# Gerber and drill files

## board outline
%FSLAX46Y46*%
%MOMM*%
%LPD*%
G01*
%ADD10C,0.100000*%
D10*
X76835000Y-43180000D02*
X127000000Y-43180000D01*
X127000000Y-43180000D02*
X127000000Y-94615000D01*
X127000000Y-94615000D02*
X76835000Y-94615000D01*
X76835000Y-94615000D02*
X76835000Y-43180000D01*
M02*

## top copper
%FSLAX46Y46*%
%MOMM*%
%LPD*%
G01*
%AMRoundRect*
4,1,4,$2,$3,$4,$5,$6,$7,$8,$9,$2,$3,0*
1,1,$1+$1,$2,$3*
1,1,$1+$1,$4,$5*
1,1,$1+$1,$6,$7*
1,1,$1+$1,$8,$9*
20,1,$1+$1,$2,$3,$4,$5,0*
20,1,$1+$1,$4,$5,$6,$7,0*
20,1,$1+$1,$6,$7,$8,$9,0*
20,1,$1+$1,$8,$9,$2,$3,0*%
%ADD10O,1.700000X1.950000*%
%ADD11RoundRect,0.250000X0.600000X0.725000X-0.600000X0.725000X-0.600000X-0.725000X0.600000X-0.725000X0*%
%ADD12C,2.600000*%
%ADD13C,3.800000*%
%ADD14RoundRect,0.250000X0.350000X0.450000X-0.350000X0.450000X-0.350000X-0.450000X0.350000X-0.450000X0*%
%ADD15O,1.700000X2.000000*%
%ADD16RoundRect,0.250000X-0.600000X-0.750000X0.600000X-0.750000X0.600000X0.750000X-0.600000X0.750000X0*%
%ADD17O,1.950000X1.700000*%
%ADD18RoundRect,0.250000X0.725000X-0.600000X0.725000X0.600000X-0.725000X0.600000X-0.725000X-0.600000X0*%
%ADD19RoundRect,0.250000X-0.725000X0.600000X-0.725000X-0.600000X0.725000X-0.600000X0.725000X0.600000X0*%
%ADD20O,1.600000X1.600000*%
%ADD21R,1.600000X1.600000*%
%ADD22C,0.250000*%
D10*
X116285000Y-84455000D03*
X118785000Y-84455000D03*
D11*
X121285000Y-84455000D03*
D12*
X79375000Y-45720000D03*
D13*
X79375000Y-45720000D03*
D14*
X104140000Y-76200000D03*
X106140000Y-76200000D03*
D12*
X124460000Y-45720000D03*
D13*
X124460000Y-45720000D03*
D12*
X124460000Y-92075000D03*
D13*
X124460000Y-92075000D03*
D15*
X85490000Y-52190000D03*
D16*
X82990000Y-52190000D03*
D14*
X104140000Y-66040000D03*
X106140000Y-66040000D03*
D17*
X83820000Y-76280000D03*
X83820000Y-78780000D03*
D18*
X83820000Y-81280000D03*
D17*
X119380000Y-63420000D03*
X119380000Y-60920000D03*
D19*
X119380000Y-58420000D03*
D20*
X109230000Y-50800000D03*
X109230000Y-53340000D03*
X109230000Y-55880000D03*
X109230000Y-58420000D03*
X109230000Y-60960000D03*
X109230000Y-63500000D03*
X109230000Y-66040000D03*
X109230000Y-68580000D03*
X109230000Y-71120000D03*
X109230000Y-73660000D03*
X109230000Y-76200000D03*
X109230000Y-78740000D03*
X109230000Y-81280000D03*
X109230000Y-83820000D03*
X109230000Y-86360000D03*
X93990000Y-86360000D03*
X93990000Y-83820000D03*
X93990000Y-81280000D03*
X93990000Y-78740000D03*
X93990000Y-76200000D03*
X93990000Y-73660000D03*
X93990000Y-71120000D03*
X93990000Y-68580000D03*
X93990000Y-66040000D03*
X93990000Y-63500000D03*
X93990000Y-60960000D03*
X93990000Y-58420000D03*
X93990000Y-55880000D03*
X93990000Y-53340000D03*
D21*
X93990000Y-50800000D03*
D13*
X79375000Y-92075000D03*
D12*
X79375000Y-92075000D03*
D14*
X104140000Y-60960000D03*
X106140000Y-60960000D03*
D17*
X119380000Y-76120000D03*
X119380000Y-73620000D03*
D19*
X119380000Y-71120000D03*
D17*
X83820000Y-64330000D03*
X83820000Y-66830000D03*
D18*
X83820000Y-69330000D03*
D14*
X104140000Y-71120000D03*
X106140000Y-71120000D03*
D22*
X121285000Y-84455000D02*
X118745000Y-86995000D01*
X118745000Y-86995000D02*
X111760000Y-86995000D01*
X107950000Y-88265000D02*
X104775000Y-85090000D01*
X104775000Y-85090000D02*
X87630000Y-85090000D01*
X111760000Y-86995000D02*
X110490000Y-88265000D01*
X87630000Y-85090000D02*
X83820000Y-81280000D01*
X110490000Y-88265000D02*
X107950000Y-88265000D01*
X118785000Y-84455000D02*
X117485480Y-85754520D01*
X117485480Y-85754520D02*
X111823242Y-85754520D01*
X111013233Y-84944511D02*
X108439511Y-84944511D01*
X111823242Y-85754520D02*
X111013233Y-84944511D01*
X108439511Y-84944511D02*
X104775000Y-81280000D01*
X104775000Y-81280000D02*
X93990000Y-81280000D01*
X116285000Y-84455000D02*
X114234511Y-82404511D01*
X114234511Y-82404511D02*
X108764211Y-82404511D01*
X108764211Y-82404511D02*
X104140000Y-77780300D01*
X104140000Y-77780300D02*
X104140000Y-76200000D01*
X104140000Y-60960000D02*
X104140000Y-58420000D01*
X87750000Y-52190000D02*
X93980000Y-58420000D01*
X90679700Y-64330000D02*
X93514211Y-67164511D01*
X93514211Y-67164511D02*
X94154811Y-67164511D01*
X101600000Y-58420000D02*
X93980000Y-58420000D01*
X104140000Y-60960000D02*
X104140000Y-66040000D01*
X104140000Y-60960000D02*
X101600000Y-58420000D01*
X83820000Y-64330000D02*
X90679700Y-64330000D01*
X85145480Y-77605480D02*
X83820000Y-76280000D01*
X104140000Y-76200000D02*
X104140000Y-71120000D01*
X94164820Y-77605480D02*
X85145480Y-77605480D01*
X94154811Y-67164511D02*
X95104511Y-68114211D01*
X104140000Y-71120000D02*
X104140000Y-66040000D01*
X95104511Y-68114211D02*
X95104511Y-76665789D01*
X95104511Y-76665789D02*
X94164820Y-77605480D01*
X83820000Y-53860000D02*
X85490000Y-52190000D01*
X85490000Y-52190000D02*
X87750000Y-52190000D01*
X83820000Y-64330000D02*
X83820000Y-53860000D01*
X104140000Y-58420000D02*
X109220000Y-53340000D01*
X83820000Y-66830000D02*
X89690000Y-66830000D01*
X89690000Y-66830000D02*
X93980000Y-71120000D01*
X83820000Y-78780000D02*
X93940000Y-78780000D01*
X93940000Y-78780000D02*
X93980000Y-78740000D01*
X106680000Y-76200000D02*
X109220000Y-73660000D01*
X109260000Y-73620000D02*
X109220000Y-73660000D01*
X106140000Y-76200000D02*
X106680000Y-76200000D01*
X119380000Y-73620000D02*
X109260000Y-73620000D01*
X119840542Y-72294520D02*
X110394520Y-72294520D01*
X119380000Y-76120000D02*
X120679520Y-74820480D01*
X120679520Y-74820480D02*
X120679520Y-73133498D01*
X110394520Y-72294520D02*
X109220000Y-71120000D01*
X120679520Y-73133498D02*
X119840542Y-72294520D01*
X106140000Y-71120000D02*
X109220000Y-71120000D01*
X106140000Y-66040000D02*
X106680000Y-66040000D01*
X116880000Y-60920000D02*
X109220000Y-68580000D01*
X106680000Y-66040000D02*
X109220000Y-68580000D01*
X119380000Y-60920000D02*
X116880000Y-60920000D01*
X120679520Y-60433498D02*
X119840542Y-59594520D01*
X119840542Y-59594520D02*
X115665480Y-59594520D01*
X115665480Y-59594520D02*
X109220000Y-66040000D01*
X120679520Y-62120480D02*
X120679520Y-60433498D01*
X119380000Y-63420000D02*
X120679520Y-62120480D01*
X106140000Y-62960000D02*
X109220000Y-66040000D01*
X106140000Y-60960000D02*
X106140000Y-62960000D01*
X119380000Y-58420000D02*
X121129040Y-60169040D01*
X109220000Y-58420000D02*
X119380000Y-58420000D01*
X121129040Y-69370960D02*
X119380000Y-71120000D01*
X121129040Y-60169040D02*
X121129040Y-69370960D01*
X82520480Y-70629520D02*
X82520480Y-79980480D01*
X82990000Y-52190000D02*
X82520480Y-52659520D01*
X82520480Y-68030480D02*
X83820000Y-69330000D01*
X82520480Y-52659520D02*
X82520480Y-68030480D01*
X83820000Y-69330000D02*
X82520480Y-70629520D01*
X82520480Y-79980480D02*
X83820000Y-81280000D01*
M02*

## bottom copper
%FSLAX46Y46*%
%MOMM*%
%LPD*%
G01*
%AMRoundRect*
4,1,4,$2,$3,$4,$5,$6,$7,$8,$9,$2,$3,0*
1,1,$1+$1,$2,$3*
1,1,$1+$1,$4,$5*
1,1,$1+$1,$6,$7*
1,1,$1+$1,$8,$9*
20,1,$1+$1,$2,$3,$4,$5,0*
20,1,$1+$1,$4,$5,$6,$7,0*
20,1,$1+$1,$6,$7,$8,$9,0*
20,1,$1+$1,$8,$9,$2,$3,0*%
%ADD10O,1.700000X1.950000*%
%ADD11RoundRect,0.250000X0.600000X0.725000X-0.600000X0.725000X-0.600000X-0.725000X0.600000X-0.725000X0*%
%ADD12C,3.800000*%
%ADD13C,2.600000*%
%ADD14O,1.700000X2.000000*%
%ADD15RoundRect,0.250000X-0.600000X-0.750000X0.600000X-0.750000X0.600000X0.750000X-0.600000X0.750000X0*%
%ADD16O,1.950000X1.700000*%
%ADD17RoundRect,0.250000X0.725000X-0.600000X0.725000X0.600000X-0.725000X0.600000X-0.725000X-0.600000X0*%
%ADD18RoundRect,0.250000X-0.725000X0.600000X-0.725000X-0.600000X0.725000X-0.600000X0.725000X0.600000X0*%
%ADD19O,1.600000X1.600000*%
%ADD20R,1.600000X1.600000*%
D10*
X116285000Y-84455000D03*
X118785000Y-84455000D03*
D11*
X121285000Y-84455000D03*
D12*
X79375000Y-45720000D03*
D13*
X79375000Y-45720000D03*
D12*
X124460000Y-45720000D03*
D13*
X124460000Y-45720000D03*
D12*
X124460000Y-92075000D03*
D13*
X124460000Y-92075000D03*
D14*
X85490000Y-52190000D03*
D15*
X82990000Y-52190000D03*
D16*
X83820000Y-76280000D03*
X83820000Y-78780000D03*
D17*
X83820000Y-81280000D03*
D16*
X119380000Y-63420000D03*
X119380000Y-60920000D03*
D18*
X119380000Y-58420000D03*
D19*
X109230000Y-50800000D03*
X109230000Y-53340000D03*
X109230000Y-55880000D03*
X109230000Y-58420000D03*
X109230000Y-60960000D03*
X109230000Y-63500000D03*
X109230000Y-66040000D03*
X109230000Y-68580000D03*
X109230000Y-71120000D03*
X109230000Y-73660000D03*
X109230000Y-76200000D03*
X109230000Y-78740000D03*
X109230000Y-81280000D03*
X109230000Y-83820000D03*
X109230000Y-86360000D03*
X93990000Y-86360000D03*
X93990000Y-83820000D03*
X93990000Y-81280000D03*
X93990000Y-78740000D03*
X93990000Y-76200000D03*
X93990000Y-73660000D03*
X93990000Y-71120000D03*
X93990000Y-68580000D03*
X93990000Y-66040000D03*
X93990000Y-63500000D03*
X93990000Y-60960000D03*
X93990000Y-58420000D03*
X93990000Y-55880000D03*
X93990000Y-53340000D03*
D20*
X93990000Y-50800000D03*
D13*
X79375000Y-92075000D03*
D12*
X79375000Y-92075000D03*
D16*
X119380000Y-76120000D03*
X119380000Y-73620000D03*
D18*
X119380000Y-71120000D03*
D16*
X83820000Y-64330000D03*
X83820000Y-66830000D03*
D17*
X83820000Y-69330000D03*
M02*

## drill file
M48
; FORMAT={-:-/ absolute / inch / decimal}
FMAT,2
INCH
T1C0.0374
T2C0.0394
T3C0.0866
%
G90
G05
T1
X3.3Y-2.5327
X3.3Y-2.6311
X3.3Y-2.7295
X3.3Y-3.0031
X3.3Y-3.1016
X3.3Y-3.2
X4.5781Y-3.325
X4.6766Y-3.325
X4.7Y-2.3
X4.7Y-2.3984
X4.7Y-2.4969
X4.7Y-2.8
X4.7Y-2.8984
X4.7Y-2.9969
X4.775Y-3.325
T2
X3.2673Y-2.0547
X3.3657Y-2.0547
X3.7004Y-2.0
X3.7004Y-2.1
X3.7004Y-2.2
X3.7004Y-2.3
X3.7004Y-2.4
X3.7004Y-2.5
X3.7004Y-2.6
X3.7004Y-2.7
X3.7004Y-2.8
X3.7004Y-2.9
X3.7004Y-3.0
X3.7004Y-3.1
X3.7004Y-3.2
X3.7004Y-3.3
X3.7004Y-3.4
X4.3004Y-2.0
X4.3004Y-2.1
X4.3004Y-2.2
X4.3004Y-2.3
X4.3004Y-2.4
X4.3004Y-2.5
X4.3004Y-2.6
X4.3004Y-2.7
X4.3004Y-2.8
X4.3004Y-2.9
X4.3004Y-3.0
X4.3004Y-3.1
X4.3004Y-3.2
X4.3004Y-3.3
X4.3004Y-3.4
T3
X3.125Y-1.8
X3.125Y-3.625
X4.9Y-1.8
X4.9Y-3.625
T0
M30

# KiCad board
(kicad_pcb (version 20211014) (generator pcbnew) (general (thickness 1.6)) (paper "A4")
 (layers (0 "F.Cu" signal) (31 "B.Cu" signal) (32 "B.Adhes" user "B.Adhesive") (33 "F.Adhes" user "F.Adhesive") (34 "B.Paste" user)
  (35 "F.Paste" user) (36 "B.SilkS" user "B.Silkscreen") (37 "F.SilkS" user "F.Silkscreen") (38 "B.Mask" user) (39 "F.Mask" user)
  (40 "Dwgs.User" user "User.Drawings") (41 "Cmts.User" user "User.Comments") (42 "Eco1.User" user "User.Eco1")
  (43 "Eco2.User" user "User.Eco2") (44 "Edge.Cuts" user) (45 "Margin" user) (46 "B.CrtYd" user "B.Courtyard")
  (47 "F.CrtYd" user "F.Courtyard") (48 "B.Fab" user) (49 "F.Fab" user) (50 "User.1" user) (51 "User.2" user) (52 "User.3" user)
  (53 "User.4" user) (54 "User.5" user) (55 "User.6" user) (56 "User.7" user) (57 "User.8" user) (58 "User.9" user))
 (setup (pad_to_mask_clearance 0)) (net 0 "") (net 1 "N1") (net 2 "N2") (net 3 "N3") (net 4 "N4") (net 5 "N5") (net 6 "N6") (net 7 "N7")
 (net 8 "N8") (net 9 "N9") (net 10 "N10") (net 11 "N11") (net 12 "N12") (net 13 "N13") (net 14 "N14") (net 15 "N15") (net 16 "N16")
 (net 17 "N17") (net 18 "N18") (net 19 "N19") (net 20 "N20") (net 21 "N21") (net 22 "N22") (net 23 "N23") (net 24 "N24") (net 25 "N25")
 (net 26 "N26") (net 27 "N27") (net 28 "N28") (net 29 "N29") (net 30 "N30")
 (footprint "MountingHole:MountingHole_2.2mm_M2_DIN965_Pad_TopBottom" (layer "F.Cu") (at 79.375 45.72)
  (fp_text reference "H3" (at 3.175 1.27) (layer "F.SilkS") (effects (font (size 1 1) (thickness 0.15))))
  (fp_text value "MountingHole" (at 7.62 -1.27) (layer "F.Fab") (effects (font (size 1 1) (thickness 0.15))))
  (pad "1" connect circle (at 0 0) (size 3.8 3.8) (layers "F.Cu" "F.Mask"))
  (pad "1" thru_hole circle (at 0 0) (size 2.6 2.6) (drill 2.2) (layers *.Cu *.Mask))
  (pad "1" connect circle (at 0 0) (size 3.8 3.8) (layers "B.Cu" "B.Mask")))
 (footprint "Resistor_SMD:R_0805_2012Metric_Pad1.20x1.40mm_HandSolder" (layer "F.Cu") (at 105.14 76.2 180)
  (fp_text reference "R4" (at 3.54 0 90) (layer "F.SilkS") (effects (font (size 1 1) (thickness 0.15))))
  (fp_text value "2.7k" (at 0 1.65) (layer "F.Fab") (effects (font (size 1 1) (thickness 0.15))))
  (pad "1" smd roundrect (at -1 0 180) (size 1.2 1.4) (layers "F.Cu" "F.Paste" "F.Mask") (roundrect_rratio 0.2083333333) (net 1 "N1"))
  (pad "2" smd roundrect (at 1 0 180) (size 1.2 1.4) (layers "F.Cu" "F.Paste" "F.Mask") (roundrect_rratio 0.2083333333) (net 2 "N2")))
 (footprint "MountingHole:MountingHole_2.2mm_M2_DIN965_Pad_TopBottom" (layer "F.Cu") (at 124.46 45.72)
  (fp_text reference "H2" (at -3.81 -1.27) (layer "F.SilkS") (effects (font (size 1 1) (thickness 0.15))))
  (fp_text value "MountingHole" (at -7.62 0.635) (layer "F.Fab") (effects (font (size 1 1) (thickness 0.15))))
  (pad "1" connect circle (at 0 0) (size 3.8 3.8) (layers "F.Cu" "F.Mask"))
  (pad "1" thru_hole circle (at 0 0) (size 2.6 2.6) (drill 2.2) (layers *.Cu *.Mask))
  (pad "1" connect circle (at 0 0) (size 3.8 3.8) (layers "B.Cu" "B.Mask")))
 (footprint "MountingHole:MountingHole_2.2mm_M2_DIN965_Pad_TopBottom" (layer "F.Cu") (at 124.46 92.075)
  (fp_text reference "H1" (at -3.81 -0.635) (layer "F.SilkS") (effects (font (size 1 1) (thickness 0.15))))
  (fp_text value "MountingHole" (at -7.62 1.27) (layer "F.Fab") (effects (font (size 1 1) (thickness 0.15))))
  (pad "1" connect circle (at 0 0) (size 3.8 3.8) (layers "F.Cu" "F.Mask"))
  (pad "1" thru_hole circle (at 0 0) (size 2.6 2.6) (drill 2.2) (layers *.Cu *.Mask))
  (pad "1" connect circle (at 0 0) (size 3.8 3.8) (layers "B.Cu" "B.Mask")))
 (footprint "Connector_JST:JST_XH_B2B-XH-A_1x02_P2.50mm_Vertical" (layer "F.Cu") (at 82.99 52.19)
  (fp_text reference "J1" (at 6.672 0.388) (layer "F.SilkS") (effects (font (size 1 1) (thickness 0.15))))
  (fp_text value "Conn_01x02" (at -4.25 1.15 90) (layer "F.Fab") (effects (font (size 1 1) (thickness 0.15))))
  (pad "1" thru_hole roundrect (at 0 0) (size 1.7 2) (drill 1) (layers *.Cu *.Mask) (roundrect_rratio 0.1470588235) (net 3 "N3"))
  (pad "2" thru_hole oval (at 2.5 0) (size 1.7 2) (drill 1) (layers *.Cu *.Mask) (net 2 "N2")))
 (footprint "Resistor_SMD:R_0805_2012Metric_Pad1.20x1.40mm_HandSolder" (layer "F.Cu") (at 105.14 66.04 180)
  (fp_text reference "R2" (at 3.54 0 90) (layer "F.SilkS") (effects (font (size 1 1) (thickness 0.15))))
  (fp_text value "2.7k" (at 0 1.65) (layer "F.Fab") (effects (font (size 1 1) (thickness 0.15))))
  (pad "1" smd roundrect (at -1 0 180) (size 1.2 1.4) (layers "F.Cu" "F.Paste" "F.Mask") (roundrect_rratio 0.2083333333) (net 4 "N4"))
  (pad "2" smd roundrect (at 1 0 180) (size 1.2 1.4) (layers "F.Cu" "F.Paste" "F.Mask") (roundrect_rratio 0.2083333333) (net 2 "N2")))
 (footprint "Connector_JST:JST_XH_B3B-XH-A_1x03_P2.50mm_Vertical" (layer "F.Cu") (at 83.82 81.28 90)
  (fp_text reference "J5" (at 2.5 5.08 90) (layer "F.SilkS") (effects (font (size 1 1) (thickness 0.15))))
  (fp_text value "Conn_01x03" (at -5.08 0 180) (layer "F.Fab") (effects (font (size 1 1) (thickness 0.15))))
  (pad "1" thru_hole roundrect (at 0 0 90) (size 1.7 1.95) (drill 0.95) (layers *.Cu *.Mask) (roundrect_rratio 0.1470588235) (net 3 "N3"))
  (pad "2" thru_hole oval (at 2.5 0 90) (size 1.7 1.95) (drill 0.95) (layers *.Cu *.Mask) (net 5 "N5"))
  (pad "3" thru_hole oval (at 5 0 90) (size 1.7 1.95) (drill 0.95) (layers *.Cu *.Mask) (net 2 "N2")))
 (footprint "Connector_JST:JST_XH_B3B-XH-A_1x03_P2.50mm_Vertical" (layer "F.Cu") (at 119.38 58.42 -90)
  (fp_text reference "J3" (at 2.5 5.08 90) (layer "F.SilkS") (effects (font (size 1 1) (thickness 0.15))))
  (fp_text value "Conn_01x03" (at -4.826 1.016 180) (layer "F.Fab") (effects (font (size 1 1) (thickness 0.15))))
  (pad "1" thru_hole roundrect (at 0 0 270) (size 1.7 1.95) (drill 0.95) (layers *.Cu *.Mask) (roundrect_rratio 0.1470588235) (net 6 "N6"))
  (pad "2" thru_hole oval (at 2.5 0 270) (size 1.7 1.95) (drill 0.95) (layers *.Cu *.Mask) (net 4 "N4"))
  (pad "3" thru_hole oval (at 5 0 270) (size 1.7 1.95) (drill 0.95) (layers *.Cu *.Mask) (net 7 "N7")))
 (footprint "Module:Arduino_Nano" (layer "F.Cu") (at 93.99 50.8)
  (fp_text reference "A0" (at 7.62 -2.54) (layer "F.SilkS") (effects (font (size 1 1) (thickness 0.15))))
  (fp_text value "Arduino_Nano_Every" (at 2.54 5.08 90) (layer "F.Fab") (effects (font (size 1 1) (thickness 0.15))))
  (pad "1" thru_hole rect (at 0 0) (size 1.6 1.6) (drill 1) (layers *.Cu *.Mask) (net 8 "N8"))
  (pad "2" thru_hole oval (at 0 2.54) (size 1.6 1.6) (drill 1) (layers *.Cu *.Mask) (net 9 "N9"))
  (pad "3" thru_hole oval (at 0 5.08) (size 1.6 1.6) (drill 1) (layers *.Cu *.Mask) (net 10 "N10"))
  (pad "4" thru_hole oval (at 0 7.62) (size 1.6 1.6) (drill 1) (layers *.Cu *.Mask) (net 2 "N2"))
  (pad "5" thru_hole oval (at 0 10.16) (size 1.6 1.6) (drill 1) (layers *.Cu *.Mask) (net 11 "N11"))
  (pad "6" thru_hole oval (at 0 12.7) (size 1.6 1.6) (drill 1) (layers *.Cu *.Mask) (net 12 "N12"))
  (pad "7" thru_hole oval (at 0 15.24) (size 1.6 1.6) (drill 1) (layers *.Cu *.Mask) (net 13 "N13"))
  (pad "8" thru_hole oval (at 0 17.78) (size 1.6 1.6) (drill 1) (layers *.Cu *.Mask) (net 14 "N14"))
  (pad "9" thru_hole oval (at 0 20.32) (size 1.6 1.6) (drill 1) (layers *.Cu *.Mask) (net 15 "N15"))
  (pad "10" thru_hole oval (at 0 22.86) (size 1.6 1.6) (drill 1) (layers *.Cu *.Mask) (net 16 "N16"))
  (pad "11" thru_hole oval (at 0 25.4) (size 1.6 1.6) (drill 1) (layers *.Cu *.Mask) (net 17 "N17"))
  (pad "12" thru_hole oval (at 0 27.94) (size 1.6 1.6) (drill 1) (layers *.Cu *.Mask) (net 5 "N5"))
  (pad "13" thru_hole oval (at 0 30.48) (size 1.6 1.6) (drill 1) (layers *.Cu *.Mask) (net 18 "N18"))
  (pad "14" thru_hole oval (at 0 33.02) (size 1.6 1.6) (drill 1) (layers *.Cu *.Mask) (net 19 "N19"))
  (pad "15" thru_hole oval (at 0 35.56) (size 1.6 1.6) (drill 1) (layers *.Cu *.Mask) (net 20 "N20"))
  (pad "16" thru_hole oval (at 15.24 35.56) (size 1.6 1.6) (drill 1) (layers *.Cu *.Mask) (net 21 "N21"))
  (pad "17" thru_hole oval (at 15.24 33.02) (size 1.6 1.6) (drill 1) (layers *.Cu *.Mask) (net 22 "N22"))
  (pad "18" thru_hole oval (at 15.24 30.48) (size 1.6 1.6) (drill 1) (layers *.Cu *.Mask) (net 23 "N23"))
  (pad "19" thru_hole oval (at 15.24 27.94) (size 1.6 1.6) (drill 1) (layers *.Cu *.Mask) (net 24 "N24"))
  (pad "20" thru_hole oval (at 15.24 25.4) (size 1.6 1.6) (drill 1) (layers *.Cu *.Mask) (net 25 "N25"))
  (pad "21" thru_hole oval (at 15.24 22.86) (size 1.6 1.6) (drill 1) (layers *.Cu *.Mask) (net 1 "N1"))
  (pad "22" thru_hole oval (at 15.24 20.32) (size 1.6 1.6) (drill 1) (layers *.Cu *.Mask) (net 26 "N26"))
  (pad "23" thru_hole oval (at 15.24 17.78) (size 1.6 1.6) (drill 1) (layers *.Cu *.Mask) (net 4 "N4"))
  (pad "24" thru_hole oval (at 15.24 15.24) (size 1.6 1.6) (drill 1) (layers *.Cu *.Mask) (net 7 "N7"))
  (pad "25" thru_hole oval (at 15.24 12.7) (size 1.6 1.6) (drill 1) (layers *.Cu *.Mask) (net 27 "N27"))
  (pad "26" thru_hole oval (at 15.24 10.16) (size 1.6 1.6) (drill 1) (layers *.Cu *.Mask) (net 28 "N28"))
  (pad "27" thru_hole oval (at 15.24 7.62) (size 1.6 1.6) (drill 1) (layers *.Cu *.Mask) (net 6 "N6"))
  (pad "28" thru_hole oval (at 15.24 5.08) (size 1.6 1.6) (drill 1) (layers *.Cu *.Mask) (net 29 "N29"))
  (pad "29" thru_hole oval (at 15.24 2.54) (size 1.6 1.6) (drill 1) (layers *.Cu *.Mask) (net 2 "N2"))
  (pad "30" thru_hole oval (at 15.24 0) (size 1.6 1.6) (drill 1) (layers *.Cu *.Mask) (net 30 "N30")))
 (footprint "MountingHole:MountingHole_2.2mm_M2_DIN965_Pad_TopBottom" (layer "F.Cu") (at 79.375 92.075)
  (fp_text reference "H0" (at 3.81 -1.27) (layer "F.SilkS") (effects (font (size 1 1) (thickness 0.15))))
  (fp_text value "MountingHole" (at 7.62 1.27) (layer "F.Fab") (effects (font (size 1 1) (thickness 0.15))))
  (pad "1" connect circle (at 0 0) (size 3.8 3.8) (layers "B.Cu" "B.Mask"))
  (pad "1" thru_hole circle (at 0 0) (size 2.6 2.6) (drill 2.2) (layers *.Cu *.Mask))
  (pad "1" connect circle (at 0 0) (size 3.8 3.8) (layers "F.Cu" "F.Mask")))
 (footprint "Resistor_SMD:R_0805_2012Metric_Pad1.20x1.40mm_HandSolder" (layer "F.Cu") (at 105.14 60.96 180)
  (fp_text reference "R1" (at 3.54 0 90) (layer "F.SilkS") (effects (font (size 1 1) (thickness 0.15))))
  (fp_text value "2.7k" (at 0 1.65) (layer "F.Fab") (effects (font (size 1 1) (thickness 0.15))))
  (pad "1" smd roundrect (at -1 0 180) (size 1.2 1.4) (layers "F.Cu" "F.Paste" "F.Mask") (roundrect_rratio 0.2083333333) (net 7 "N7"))
  (pad "2" smd roundrect (at 1 0 180) (size 1.2 1.4) (layers "F.Cu" "F.Paste" "F.Mask") (roundrect_rratio 0.2083333333) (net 2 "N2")))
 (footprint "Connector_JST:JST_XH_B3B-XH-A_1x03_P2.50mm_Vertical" (layer "F.Cu") (at 119.38 71.12 -90)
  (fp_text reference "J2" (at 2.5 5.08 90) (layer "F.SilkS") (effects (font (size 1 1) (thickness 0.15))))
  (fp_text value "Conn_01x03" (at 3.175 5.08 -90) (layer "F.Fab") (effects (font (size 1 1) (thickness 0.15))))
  (pad "1" thru_hole roundrect (at 0 0 270) (size 1.7 1.95) (drill 0.95) (layers *.Cu *.Mask) (roundrect_rratio 0.1470588235) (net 6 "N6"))
  (pad "2" thru_hole oval (at 2.5 0 270) (size 1.7 1.95) (drill 0.95) (layers *.Cu *.Mask) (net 1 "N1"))
  (pad "3" thru_hole oval (at 5 0 270) (size 1.7 1.95) (drill 0.95) (layers *.Cu *.Mask) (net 26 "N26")))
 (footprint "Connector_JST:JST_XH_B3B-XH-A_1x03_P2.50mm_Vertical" (layer "F.Cu") (at 83.82 69.33 90)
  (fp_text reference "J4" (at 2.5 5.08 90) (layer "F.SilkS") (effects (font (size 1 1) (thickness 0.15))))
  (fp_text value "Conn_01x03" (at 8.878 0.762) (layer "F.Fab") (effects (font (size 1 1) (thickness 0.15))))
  (pad "1" thru_hole roundrect (at 0 0 90) (size 1.7 1.95) (drill 0.95) (layers *.Cu *.Mask) (roundrect_rratio 0.1470588235) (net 3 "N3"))
  (pad "2" thru_hole oval (at 2.5 0 90) (size 1.7 1.95) (drill 0.95) (layers *.Cu *.Mask) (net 15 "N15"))
  (pad "3" thru_hole oval (at 5 0 90) (size 1.7 1.95) (drill 0.95) (layers *.Cu *.Mask) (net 2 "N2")))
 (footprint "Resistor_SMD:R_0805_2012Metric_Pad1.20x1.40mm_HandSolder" (layer "F.Cu") (at 105.14 71.12 180)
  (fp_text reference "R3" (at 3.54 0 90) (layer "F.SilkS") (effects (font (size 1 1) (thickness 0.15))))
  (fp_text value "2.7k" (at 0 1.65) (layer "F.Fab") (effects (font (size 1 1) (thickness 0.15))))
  (pad "1" smd roundrect (at -1 0 180) (size 1.2 1.4) (layers "F.Cu" "F.Paste" "F.Mask") (roundrect_rratio 0.2083333333) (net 26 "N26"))
  (pad "2" smd roundrect (at 1 0 180) (size 1.2 1.4) (layers "F.Cu" "F.Paste" "F.Mask") (roundrect_rratio 0.2083333333) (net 2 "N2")))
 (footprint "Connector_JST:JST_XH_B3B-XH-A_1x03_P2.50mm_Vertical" (layer "F.Cu") (at 121.285 84.455 180)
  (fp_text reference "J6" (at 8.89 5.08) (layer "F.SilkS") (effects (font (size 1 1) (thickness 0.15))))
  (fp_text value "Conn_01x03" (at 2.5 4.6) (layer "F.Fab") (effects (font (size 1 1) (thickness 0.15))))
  (pad "1" thru_hole roundrect (at 0 0 180) (size 1.7 1.95) (drill 0.95) (layers *.Cu *.Mask) (roundrect_rratio 0.1470588235) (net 3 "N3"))
  (pad "2" thru_hole oval (at 2.5 0 180) (size 1.7 1.95) (drill 0.95) (layers *.Cu *.Mask) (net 18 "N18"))
  (pad "3" thru_hole oval (at 5 0 180) (size 1.7 1.95) (drill 0.95) (layers *.Cu *.Mask) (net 2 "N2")))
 (gr_rect (start 76.835 43.18) (end 127 94.615) (layer "Edge.Cuts") (width 0.1) (fill none))
 (segment (start 108.764211 82.404511) (end 104.14 77.7803) (width 0.25) (layer "F.Cu") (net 2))
 (segment (start 114.234511 82.404511) (end 108.764211 82.404511) (width 0.25) (layer "F.Cu") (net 2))
 (segment (start 104.14 60.96) (end 104.14 58.42) (width 0.25) (layer "F.Cu") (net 2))
 (segment (start 87.75 52.19) (end 93.98 58.42) (width 0.25) (layer "F.Cu") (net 2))
 (segment (start 90.6797 64.33) (end 93.514211 67.164511) (width 0.25) (layer "F.Cu") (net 2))
 (segment (start 93.514211 67.164511) (end 94.154811 67.164511) (width 0.25) (layer "F.Cu") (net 2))
 (segment (start 101.6 58.42) (end 93.98 58.42) (width 0.25) (layer "F.Cu") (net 2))
 (segment (start 104.14 60.96) (end 104.14 66.04) (width 0.25) (layer "F.Cu") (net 2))
 (segment (start 104.14 60.96) (end 101.6 58.42) (width 0.25) (layer "F.Cu") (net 2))
 (segment (start 83.82 64.33) (end 90.6797 64.33) (width 0.25) (layer "F.Cu") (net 2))
 (segment (start 85.14548 77.60548) (end 83.82 76.28) (width 0.25) (layer "F.Cu") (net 2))
 (segment (start 104.14 76.2) (end 104.14 71.12) (width 0.25) (layer "F.Cu") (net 2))
 (segment (start 94.16482 77.60548) (end 85.14548 77.60548) (width 0.25) (layer "F.Cu") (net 2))
 (segment (start 94.154811 67.164511) (end 95.104511 68.114211) (width 0.25) (layer "F.Cu") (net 2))
 (segment (start 116.285 84.455) (end 114.234511 82.404511) (width 0.25) (layer "F.Cu") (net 2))
 (segment (start 104.14 71.12) (end 104.14 66.04) (width 0.25) (layer "F.Cu") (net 2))
 (segment (start 95.104511 68.114211) (end 95.104511 76.665789) (width 0.25) (layer "F.Cu") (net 2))
 (segment (start 95.104511 76.665789) (end 94.16482 77.60548) (width 0.25) (layer "F.Cu") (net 2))
 (segment (start 83.82 53.86) (end 85.49 52.19) (width 0.25) (layer "F.Cu") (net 2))
 (segment (start 85.49 52.19) (end 87.75 52.19) (width 0.25) (layer "F.Cu") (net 2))
 (segment (start 104.14 77.7803) (end 104.14 76.2) (width 0.25) (layer "F.Cu") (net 2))
 (segment (start 83.82 64.33) (end 83.82 53.86) (width 0.25) (layer "F.Cu") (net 2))
 (segment (start 104.14 58.42) (end 109.22 53.34) (width 0.25) (layer "F.Cu") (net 2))
 (segment (start 83.82 66.83) (end 89.69 66.83) (width 0.25) (layer "F.Cu") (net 15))
 (segment (start 89.69 66.83) (end 93.98 71.12) (width 0.25) (layer "F.Cu") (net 15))
 (segment (start 83.82 78.78) (end 93.94 78.78) (width 0.25) (layer "F.Cu") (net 5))
 (segment (start 93.94 78.78) (end 93.98 78.74) (width 0.25) (layer "F.Cu") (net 5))
 (segment (start 108.439511 84.944511) (end 104.775 81.28) (width 0.25) (layer "F.Cu") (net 18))
 (segment (start 104.775 81.28) (end 93.99 81.28) (width 0.25) (layer "F.Cu") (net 18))
 (segment (start 118.785 84.455) (end 117.48548 85.75452) (width 0.25) (layer "F.Cu") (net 18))
 (segment (start 111.823242 85.75452) (end 111.013233 84.944511) (width 0.25) (layer "F.Cu") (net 18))
 (segment (start 117.48548 85.75452) (end 111.823242 85.75452) (width 0.25) (layer "F.Cu") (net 18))
 (segment (start 111.013233 84.944511) (end 108.439511 84.944511) (width 0.25) (layer "F.Cu") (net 18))
 (segment (start 106.68 76.2) (end 109.22 73.66) (width 0.25) (layer "F.Cu") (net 1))
 (segment (start 109.26 73.62) (end 109.22 73.66) (width 0.25) (layer "F.Cu") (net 1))
 (segment (start 106.14 76.2) (end 106.68 76.2) (width 0.25) (layer "F.Cu") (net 1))
 (segment (start 119.38 73.62) (end 109.26 73.62) (width 0.25) (layer "F.Cu") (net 1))
 (segment (start 119.840542 72.29452) (end 110.39452 72.29452) (width 0.25) (layer "F.Cu") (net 26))
 (segment (start 119.38 76.12) (end 120.67952 74.82048) (width 0.25) (layer "F.Cu") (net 26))
 (segment (start 120.67952 74.82048) (end 120.67952 73.133498) (width 0.25) (layer "F.Cu") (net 26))
 (segment (start 110.39452 72.29452) (end 109.22 71.12) (width 0.25) (layer "F.Cu") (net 26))
 (segment (start 120.67952 73.133498) (end 119.840542 72.29452) (width 0.25) (layer "F.Cu") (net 26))
 (segment (start 106.14 71.12) (end 109.22 71.12) (width 0.25) (layer "F.Cu") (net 26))
 (segment (start 106.14 66.04) (end 106.68 66.04) (width 0.25) (layer "F.Cu") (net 4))
 (segment (start 116.88 60.92) (end 109.22 68.58) (width 0.25) (layer "F.Cu") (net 4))
 (segment (start 106.68 66.04) (end 109.22 68.58) (width 0.25) (layer "F.Cu") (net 4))
 (segment (start 119.38 60.92) (end 116.88 60.92) (width 0.25) (layer "F.Cu") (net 4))
 (segment (start 120.67952 60.433498) (end 119.840542 59.59452) (width 0.25) (layer "F.Cu") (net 7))
 (segment (start 119.840542 59.59452) (end 115.66548 59.59452) (width 0.25) (layer "F.Cu") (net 7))
 (segment (start 115.66548 59.59452) (end 109.22 66.04) (width 0.25) (layer "F.Cu") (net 7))
 (segment (start 120.67952 62.12048) (end 120.67952 60.433498) (width 0.25) (layer "F.Cu") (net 7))
 (segment (start 119.38 63.42) (end 120.67952 62.12048) (width 0.25) (layer "F.Cu") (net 7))
 (segment (start 106.14 62.96) (end 109.22 66.04) (width 0.25) (layer "F.Cu") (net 7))
 (segment (start 106.14 60.96) (end 106.14 62.96) (width 0.25) (layer "F.Cu") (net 7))
 (segment (start 119.38 58.42) (end 121.12904 60.16904) (width 0.25) (layer "F.Cu") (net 6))
 (segment (start 109.22 58.42) (end 119.38 58.42) (width 0.25) (layer "F.Cu") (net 6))
 (segment (start 121.12904 69.37096) (end 119.38 71.12) (width 0.25) (layer "F.Cu") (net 6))
 (segment (start 121.12904 60.16904) (end 121.12904 69.37096) (width 0.25) (layer "F.Cu") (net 6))
 (segment (start 82.52048 70.62952) (end 82.52048 79.98048) (width 0.25) (layer "F.Cu") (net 3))
 (segment (start 87.63 85.09) (end 83.82 81.28) (width 0.25) (layer "F.Cu") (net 3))
 (segment (start 82.99 52.19) (end 82.52048 52.65952) (width 0.25) (layer "F.Cu") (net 3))
 (segment (start 121.285 84.455) (end 118.745 86.995) (width 0.25) (layer "F.Cu") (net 3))
 (segment (start 82.52048 68.03048) (end 83.82 69.33) (width 0.25) (layer "F.Cu") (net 3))
 (segment (start 82.52048 52.65952) (end 82.52048 68.03048) (width 0.25) (layer "F.Cu") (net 3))
 (segment (start 83.82 69.33) (end 82.52048 70.62952) (width 0.25) (layer "F.Cu") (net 3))
 (segment (start 110.49 88.265) (end 107.95 88.265) (width 0.25) (layer "F.Cu") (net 3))
 (segment (start 111.76 86.995) (end 110.49 88.265) (width 0.25) (layer "F.Cu") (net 3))
 (segment (start 82.52048 79.98048) (end 83.82 81.28) (width 0.25) (layer "F.Cu") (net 3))
 (segment (start 104.775 85.09) (end 87.63 85.09) (width 0.25) (layer "F.Cu") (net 3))
 (segment (start 118.745 86.995) (end 111.76 86.995) (width 0.25) (layer "F.Cu") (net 3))
 (segment (start 107.95 88.265) (end 104.775 85.09) (width 0.25) (layer "F.Cu") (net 3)))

